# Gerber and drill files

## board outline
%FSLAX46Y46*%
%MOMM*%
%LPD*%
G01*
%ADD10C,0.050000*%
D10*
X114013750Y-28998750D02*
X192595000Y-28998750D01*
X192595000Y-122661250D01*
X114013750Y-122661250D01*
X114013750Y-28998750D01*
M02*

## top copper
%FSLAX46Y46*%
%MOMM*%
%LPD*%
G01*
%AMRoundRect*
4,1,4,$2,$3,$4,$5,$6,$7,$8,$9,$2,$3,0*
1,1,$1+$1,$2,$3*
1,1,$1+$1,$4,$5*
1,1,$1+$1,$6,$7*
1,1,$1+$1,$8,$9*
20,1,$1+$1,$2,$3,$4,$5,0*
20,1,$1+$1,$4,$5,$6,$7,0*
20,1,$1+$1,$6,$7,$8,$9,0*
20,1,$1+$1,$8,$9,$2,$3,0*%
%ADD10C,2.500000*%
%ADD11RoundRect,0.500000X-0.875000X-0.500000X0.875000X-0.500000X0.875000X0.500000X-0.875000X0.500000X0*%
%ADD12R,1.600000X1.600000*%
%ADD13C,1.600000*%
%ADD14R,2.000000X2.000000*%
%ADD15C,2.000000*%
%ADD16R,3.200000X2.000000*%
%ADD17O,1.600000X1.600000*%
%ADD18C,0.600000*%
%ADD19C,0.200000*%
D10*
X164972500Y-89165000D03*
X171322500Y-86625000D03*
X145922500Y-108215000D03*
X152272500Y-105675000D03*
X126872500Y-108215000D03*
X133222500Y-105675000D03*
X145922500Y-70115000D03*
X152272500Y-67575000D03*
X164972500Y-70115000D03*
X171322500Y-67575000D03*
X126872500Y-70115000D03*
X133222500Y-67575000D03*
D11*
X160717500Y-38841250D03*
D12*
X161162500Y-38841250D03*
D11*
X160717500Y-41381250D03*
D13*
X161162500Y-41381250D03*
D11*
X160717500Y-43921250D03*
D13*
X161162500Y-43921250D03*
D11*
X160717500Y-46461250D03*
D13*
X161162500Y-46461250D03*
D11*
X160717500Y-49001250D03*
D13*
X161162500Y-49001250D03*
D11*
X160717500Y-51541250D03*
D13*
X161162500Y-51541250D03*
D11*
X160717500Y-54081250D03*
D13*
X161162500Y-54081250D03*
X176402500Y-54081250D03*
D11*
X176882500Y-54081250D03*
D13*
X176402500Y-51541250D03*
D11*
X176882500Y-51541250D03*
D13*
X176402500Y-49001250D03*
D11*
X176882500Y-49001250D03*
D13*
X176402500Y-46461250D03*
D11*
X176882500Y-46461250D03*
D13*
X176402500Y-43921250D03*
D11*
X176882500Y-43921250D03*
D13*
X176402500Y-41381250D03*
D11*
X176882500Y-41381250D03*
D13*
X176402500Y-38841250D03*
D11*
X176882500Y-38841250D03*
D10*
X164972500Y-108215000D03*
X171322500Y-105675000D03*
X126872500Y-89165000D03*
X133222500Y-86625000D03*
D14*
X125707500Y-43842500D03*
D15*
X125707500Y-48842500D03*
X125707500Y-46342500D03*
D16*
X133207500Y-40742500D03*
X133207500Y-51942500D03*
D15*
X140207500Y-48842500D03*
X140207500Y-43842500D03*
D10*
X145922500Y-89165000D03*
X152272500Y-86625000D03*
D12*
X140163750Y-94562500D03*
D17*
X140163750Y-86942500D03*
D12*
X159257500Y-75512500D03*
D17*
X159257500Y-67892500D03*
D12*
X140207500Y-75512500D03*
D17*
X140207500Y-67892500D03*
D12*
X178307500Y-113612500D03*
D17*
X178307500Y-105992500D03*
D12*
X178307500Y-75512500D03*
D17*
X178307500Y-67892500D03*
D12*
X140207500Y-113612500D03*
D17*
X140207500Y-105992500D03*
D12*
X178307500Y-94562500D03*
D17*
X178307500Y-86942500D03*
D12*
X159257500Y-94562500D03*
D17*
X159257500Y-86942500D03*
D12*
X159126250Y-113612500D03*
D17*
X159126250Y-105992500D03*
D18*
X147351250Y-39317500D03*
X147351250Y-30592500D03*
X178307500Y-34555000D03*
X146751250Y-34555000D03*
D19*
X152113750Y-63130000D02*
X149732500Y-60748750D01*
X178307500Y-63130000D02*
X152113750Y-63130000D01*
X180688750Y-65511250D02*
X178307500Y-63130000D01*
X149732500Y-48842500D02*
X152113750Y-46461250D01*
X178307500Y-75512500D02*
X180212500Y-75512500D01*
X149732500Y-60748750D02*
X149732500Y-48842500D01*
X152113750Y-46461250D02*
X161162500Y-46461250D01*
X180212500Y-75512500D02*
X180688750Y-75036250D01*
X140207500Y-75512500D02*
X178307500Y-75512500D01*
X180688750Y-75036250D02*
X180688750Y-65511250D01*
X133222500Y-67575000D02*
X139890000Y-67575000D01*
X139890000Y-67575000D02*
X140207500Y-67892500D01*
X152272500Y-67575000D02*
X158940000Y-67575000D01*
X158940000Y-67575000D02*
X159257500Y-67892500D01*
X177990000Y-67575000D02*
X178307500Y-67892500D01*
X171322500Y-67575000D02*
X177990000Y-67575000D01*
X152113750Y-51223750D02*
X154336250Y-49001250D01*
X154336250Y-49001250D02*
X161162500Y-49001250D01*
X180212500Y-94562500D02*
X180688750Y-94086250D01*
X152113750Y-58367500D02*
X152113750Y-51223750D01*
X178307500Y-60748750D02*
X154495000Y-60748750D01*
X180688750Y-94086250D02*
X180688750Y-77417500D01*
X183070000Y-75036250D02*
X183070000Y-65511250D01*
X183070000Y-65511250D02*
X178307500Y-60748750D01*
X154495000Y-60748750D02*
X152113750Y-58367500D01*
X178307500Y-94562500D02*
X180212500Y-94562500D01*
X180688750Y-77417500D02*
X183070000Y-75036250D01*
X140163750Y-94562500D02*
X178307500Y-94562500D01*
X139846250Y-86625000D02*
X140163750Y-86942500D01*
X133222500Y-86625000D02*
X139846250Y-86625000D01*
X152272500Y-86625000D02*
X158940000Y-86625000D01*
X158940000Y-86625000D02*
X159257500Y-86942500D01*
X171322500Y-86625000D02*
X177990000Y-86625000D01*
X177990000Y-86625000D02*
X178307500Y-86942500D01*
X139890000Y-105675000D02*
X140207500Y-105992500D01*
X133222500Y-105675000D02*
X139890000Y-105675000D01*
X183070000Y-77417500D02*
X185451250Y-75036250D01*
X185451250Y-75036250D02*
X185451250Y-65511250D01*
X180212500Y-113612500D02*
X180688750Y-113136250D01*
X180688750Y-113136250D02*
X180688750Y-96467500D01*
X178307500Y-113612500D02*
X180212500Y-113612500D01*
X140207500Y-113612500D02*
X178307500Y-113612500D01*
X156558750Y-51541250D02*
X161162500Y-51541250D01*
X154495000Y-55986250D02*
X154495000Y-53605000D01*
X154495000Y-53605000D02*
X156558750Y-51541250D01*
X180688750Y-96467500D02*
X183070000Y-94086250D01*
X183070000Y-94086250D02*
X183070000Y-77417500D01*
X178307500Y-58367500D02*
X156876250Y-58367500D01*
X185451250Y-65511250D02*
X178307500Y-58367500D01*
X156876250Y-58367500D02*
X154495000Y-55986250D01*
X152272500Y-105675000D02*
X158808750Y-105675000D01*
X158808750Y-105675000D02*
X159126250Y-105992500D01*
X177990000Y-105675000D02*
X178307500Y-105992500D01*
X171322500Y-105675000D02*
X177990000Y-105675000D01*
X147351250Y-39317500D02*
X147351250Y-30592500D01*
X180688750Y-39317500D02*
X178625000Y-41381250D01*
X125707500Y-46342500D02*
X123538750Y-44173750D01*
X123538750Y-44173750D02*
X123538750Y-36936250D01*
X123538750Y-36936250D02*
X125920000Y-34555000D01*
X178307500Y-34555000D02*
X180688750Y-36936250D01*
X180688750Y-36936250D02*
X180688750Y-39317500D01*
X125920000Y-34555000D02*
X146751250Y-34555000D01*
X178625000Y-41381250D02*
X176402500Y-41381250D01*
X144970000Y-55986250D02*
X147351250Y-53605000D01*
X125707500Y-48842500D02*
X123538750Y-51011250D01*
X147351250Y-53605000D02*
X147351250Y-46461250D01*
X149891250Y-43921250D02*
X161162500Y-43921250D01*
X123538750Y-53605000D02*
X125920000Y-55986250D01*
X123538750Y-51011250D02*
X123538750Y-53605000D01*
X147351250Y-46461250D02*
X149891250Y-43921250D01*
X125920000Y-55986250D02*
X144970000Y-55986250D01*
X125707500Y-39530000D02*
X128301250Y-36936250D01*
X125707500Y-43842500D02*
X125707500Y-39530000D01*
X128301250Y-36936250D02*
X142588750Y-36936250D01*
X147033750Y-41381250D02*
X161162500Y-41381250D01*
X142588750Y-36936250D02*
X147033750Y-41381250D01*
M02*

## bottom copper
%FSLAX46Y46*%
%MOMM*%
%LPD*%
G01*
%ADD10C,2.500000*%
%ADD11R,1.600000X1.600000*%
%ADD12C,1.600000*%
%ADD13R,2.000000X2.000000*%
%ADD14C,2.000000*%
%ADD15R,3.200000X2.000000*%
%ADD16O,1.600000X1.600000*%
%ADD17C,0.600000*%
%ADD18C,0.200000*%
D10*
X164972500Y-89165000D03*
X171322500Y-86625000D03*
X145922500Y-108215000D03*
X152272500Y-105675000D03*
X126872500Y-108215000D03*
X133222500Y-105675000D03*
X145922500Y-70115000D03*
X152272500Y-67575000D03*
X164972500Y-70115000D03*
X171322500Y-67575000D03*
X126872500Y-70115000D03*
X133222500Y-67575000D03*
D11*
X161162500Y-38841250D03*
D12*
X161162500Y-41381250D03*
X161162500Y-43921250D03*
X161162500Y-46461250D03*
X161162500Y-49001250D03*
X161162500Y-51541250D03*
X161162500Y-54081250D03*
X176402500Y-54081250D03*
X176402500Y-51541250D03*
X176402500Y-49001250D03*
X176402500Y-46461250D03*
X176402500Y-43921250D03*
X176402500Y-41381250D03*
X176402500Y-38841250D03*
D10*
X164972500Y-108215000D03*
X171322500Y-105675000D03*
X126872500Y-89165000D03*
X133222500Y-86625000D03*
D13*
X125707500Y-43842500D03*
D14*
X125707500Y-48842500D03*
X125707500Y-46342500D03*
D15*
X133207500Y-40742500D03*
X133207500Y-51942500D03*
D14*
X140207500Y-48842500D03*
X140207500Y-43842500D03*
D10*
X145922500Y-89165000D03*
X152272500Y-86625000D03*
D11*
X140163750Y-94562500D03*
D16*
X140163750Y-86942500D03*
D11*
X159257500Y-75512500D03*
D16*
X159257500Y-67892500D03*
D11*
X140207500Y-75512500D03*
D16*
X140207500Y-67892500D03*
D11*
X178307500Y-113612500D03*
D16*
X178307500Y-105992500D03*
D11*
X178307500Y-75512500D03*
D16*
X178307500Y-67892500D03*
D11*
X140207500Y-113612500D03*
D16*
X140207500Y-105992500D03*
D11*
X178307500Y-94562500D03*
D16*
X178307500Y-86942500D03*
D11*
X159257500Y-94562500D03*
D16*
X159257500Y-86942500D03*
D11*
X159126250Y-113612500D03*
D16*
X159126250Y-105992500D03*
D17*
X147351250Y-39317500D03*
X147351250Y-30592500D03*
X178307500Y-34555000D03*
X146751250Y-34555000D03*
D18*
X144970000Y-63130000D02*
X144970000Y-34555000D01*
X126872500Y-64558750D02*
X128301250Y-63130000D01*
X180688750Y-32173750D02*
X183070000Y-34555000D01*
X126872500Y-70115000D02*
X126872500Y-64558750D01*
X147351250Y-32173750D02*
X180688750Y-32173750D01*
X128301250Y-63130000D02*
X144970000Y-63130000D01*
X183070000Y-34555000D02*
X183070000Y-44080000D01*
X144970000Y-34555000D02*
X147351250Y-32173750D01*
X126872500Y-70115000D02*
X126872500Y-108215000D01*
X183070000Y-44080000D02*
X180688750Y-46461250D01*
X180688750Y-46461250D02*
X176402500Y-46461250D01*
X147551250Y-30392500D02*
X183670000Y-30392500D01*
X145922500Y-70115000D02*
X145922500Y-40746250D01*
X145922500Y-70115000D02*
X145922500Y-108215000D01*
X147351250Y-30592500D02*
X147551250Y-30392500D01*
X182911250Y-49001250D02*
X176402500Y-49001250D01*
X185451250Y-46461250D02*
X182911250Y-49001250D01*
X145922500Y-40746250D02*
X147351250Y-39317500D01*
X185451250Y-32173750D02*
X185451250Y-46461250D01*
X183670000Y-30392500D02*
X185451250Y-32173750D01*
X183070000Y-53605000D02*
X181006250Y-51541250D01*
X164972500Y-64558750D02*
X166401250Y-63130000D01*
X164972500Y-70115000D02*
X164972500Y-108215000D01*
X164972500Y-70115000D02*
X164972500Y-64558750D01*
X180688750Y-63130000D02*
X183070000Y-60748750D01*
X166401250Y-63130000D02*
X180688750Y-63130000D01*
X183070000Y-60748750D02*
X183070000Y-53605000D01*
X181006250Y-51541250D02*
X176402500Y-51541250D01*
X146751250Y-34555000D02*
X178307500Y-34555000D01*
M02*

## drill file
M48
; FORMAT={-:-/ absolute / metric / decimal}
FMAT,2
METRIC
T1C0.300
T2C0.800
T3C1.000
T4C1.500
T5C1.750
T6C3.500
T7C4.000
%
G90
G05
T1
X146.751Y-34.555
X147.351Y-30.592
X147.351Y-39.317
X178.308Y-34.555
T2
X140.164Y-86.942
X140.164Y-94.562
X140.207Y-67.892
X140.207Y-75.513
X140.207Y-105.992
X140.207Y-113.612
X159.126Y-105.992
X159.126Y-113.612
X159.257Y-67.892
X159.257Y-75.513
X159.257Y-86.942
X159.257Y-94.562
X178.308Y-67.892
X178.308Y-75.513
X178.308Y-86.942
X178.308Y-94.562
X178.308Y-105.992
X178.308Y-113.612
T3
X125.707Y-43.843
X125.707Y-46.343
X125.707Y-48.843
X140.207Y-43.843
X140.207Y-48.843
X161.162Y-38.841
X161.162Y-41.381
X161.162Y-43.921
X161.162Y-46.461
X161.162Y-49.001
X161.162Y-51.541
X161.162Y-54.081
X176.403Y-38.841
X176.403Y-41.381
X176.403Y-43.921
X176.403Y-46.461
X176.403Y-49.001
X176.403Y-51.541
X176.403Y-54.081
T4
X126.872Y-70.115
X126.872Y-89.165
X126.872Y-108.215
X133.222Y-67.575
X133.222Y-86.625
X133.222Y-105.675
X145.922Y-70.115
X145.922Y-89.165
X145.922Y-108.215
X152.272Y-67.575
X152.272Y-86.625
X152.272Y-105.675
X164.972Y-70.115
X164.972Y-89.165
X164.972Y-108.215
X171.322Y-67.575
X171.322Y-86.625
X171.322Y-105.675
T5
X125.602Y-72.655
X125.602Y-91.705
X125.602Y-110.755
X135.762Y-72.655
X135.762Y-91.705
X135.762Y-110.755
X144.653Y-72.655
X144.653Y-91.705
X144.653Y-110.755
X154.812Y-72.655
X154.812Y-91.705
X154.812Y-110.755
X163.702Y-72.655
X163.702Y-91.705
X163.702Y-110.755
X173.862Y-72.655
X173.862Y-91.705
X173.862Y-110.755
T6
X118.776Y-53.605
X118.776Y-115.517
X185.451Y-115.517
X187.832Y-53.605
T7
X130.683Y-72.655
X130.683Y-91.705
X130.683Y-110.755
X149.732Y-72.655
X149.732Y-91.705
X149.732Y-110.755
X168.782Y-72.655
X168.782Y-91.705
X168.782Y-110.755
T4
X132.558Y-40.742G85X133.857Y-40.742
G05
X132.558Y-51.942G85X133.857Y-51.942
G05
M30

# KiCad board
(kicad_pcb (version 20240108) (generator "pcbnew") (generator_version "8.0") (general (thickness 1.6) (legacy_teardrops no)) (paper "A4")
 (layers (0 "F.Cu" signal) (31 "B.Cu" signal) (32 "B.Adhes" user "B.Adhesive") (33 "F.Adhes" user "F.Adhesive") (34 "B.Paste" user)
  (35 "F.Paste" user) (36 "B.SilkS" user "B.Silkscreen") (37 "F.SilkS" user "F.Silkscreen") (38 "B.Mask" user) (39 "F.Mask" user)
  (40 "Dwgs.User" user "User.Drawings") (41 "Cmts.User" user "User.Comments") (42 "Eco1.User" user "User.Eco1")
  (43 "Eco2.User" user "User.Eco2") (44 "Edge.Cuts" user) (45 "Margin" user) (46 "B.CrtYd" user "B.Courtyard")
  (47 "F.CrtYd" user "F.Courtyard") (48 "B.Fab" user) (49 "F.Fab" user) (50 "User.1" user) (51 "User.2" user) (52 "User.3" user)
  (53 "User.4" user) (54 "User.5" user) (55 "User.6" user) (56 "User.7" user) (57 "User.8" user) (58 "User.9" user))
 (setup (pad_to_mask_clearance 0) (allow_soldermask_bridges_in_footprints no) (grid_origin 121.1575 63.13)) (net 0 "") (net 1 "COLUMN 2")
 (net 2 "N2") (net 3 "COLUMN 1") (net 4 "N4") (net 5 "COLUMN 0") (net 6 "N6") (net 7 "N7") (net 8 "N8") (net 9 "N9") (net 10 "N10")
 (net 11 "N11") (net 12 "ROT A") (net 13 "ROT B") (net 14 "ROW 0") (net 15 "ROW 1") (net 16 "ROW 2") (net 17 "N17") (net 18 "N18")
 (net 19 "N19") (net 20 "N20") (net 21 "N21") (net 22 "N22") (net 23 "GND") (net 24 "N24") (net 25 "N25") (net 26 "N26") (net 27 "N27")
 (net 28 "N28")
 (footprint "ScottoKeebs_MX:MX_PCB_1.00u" (layer "F.Cu") (at 168.7825 91.705)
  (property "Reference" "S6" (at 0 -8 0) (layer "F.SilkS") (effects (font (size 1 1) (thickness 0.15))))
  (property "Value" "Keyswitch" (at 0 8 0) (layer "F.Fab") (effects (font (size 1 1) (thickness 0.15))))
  (pad "" np_thru_hole circle (at -5.08 0) (size 1.75 1.75) (drill 1.75) (layers "*.Cu" "*.Mask"))
  (pad "" np_thru_hole circle (at 0 0) (size 4 4) (drill 4) (layers "*.Cu" "*.Mask"))
  (pad "" np_thru_hole circle (at 5.08 0) (size 1.75 1.75) (drill 1.75) (layers "*.Cu" "*.Mask"))
  (pad "1" thru_hole circle (at -3.81 -2.54) (size 2.5 2.5) (drill 1.5) (layers "*.Cu" "*.Mask") (remove_unused_layers no)
   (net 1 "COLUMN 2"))
  (pad "2" thru_hole circle (at 2.54 -5.08) (size 2.5 2.5) (drill 1.5) (layers "*.Cu" "*.Mask") (remove_unused_layers no) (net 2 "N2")))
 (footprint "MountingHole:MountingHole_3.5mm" (layer "F.Cu") (at 118.77625 53.605)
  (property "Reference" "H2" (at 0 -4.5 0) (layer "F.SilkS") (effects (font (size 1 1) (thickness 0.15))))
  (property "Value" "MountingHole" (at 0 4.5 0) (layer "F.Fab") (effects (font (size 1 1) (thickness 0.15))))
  (pad "" np_thru_hole circle (at 0 0) (size 3.5 3.5) (drill 3.5) (layers "*.Cu" "*.Mask")))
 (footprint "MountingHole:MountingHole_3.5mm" (layer "F.Cu") (at 118.77625 115.5175)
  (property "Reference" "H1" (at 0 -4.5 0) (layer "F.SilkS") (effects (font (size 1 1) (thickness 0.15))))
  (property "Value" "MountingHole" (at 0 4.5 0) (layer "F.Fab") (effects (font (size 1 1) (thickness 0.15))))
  (pad "" np_thru_hole circle (at 0 0) (size 3.5 3.5) (drill 3.5) (layers "*.Cu" "*.Mask")))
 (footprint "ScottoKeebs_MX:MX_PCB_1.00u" (layer "F.Cu") (at 149.7325 110.755)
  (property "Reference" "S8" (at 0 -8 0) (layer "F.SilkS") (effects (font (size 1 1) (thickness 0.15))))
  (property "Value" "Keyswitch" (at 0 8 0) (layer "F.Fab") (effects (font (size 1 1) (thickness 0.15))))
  (pad "" np_thru_hole circle (at -5.08 0) (size 1.75 1.75) (drill 1.75) (layers "*.Cu" "*.Mask"))
  (pad "" np_thru_hole circle (at 0 0) (size 4 4) (drill 4) (layers "*.Cu" "*.Mask"))
  (pad "" np_thru_hole circle (at 5.08 0) (size 1.75 1.75) (drill 1.75) (layers "*.Cu" "*.Mask"))
  (pad "1" thru_hole circle (at -3.81 -2.54) (size 2.5 2.5) (drill 1.5) (layers "*.Cu" "*.Mask") (remove_unused_layers no)
   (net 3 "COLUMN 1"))
  (pad "2" thru_hole circle (at 2.54 -5.08) (size 2.5 2.5) (drill 1.5) (layers "*.Cu" "*.Mask") (remove_unused_layers no) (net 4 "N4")))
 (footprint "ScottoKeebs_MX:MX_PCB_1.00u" (layer "F.Cu") (at 130.6825 110.755)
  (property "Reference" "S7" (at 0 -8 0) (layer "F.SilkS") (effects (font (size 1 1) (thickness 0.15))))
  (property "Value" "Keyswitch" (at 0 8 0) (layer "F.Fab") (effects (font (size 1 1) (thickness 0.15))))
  (pad "" np_thru_hole circle (at -5.08 0) (size 1.75 1.75) (drill 1.75) (layers "*.Cu" "*.Mask"))
  (pad "" np_thru_hole circle (at 0 0) (size 4 4) (drill 4) (layers "*.Cu" "*.Mask"))
  (pad "" np_thru_hole circle (at 5.08 0) (size 1.75 1.75) (drill 1.75) (layers "*.Cu" "*.Mask"))
  (pad "1" thru_hole circle (at -3.81 -2.54) (size 2.5 2.5) (drill 1.5) (layers "*.Cu" "*.Mask") (remove_unused_layers no)
   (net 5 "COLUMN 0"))
  (pad "2" thru_hole circle (at 2.54 -5.08) (size 2.5 2.5) (drill 1.5) (layers "*.Cu" "*.Mask") (remove_unused_layers no) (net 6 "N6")))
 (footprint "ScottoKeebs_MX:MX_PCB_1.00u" (layer "F.Cu") (at 149.7325 72.655)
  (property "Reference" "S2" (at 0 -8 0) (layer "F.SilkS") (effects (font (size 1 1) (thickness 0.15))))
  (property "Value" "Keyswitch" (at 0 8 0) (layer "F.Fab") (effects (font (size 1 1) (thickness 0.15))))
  (pad "" np_thru_hole circle (at -5.08 0) (size 1.75 1.75) (drill 1.75) (layers "*.Cu" "*.Mask"))
  (pad "" np_thru_hole circle (at 0 0) (size 4 4) (drill 4) (layers "*.Cu" "*.Mask"))
  (pad "" np_thru_hole circle (at 5.08 0) (size 1.75 1.75) (drill 1.75) (layers "*.Cu" "*.Mask"))
  (pad "1" thru_hole circle (at -3.81 -2.54) (size 2.5 2.5) (drill 1.5) (layers "*.Cu" "*.Mask") (remove_unused_layers no)
   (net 3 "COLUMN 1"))
  (pad "2" thru_hole circle (at 2.54 -5.08) (size 2.5 2.5) (drill 1.5) (layers "*.Cu" "*.Mask") (remove_unused_layers no) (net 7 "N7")))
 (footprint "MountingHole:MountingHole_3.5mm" (layer "F.Cu") (at 187.8325 53.605)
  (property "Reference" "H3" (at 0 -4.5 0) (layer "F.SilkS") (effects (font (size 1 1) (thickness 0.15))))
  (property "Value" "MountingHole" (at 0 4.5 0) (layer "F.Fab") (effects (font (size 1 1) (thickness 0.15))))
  (pad "" np_thru_hole circle (at 0 0) (size 3.5 3.5) (drill 3.5) (layers "*.Cu" "*.Mask")))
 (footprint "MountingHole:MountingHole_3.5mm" (layer "F.Cu") (at 185.45125 115.5175)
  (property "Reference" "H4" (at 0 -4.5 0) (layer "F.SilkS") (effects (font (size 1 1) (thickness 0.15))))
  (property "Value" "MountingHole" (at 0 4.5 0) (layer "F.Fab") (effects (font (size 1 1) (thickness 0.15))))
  (pad "" np_thru_hole circle (at 0 0) (size 3.5 3.5) (drill 3.5) (layers "*.Cu" "*.Mask")))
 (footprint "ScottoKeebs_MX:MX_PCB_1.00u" (layer "F.Cu") (at 168.7825 72.655)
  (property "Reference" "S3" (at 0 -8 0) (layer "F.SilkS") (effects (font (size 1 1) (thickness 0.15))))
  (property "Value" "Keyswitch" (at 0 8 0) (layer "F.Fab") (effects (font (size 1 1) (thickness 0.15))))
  (pad "" np_thru_hole circle (at -5.08 0) (size 1.75 1.75) (drill 1.75) (layers "*.Cu" "*.Mask"))
  (pad "" np_thru_hole circle (at 0 0) (size 4 4) (drill 4) (layers "*.Cu" "*.Mask"))
  (pad "" np_thru_hole circle (at 5.08 0) (size 1.75 1.75) (drill 1.75) (layers "*.Cu" "*.Mask"))
  (pad "1" thru_hole circle (at -3.81 -2.54) (size 2.5 2.5) (drill 1.5) (layers "*.Cu" "*.Mask") (remove_unused_layers no)
   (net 1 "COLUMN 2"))
  (pad "2" thru_hole circle (at 2.54 -5.08) (size 2.5 2.5) (drill 1.5) (layers "*.Cu" "*.Mask") (remove_unused_layers no) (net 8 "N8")))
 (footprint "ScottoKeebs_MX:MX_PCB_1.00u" (layer "F.Cu") (at 130.6825 72.655)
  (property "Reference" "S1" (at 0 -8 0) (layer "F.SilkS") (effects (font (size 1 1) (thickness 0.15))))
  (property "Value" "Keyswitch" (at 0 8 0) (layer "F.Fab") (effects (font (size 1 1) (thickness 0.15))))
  (pad "" np_thru_hole circle (at -5.08 0) (size 1.75 1.75) (drill 1.75) (layers "*.Cu" "*.Mask"))
  (pad "" np_thru_hole circle (at 0 0) (size 4 4) (drill 4) (layers "*.Cu" "*.Mask"))
  (pad "" np_thru_hole circle (at 5.08 0) (size 1.75 1.75) (drill 1.75) (layers "*.Cu" "*.Mask"))
  (pad "1" thru_hole circle (at -3.81 -2.54) (size 2.5 2.5) (drill 1.5) (layers "*.Cu" "*.Mask") (remove_unused_layers no)
   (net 5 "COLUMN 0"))
  (pad "2" thru_hole circle (at 2.54 -5.08) (size 2.5 2.5) (drill 1.5) (layers "*.Cu" "*.Mask") (remove_unused_layers no) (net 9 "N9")))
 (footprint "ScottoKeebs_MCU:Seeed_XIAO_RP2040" (layer "F.Cu") (at 168.7825 46.46125)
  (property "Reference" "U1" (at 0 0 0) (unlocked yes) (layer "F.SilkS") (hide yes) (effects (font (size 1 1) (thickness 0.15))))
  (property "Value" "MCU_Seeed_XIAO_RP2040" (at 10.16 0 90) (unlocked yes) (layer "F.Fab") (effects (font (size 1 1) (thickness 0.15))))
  (pad "1" smd roundrect (at -8.065 -7.62) (size 2.75 2) (layers "F.Cu" "F.Paste" "F.Mask") (roundrect_rratio 0.25) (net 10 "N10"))
  (pad "1" thru_hole rect (at -7.62 -7.62 90) (size 1.6 1.6) (drill 1) (layers "*.Cu" "*.Mask") (remove_unused_layers no) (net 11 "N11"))
  (pad "2" smd roundrect (at -8.065 -5.08) (size 2.75 2) (layers "F.Cu" "F.Paste" "F.Mask") (roundrect_rratio 0.25) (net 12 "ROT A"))
  (pad "2" thru_hole circle (at -7.62 -5.08 90) (size 1.6 1.6) (drill 1) (layers "*.Cu" "*.Mask") (remove_unused_layers no) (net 12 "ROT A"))
  (pad "3" smd roundrect (at -8.065 -2.54) (size 2.75 2) (layers "F.Cu" "F.Paste" "F.Mask") (roundrect_rratio 0.25) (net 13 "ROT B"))
  (pad "3" thru_hole circle (at -7.62 -2.54 90) (size 1.6 1.6) (drill 1) (layers "*.Cu" "*.Mask") (remove_unused_layers no) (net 13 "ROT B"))
  (pad "4" smd roundrect (at -8.065 0) (size 2.75 2) (layers "F.Cu" "F.Paste" "F.Mask") (roundrect_rratio 0.25) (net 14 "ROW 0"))
  (pad "4" thru_hole circle (at -7.62 0 90) (size 1.6 1.6) (drill 1) (layers "*.Cu" "*.Mask") (remove_unused_layers no) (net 14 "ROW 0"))
  (pad "5" smd roundrect (at -8.065 2.54) (size 2.75 2) (layers "F.Cu" "F.Paste" "F.Mask") (roundrect_rratio 0.25) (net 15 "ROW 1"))
  (pad "5" thru_hole circle (at -7.62 2.54 90) (size 1.6 1.6) (drill 1) (layers "*.Cu" "*.Mask") (remove_unused_layers no) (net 15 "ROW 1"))
  (pad "6" smd roundrect (at -8.065 5.08) (size 2.75 2) (layers "F.Cu" "F.Paste" "F.Mask") (roundrect_rratio 0.25) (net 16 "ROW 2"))
  (pad "6" thru_hole circle (at -7.62 5.08 90) (size 1.6 1.6) (drill 1) (layers "*.Cu" "*.Mask") (remove_unused_layers no) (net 16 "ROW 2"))
  (pad "7" smd roundrect (at -8.065 7.62) (size 2.75 2) (layers "F.Cu" "F.Paste" "F.Mask") (roundrect_rratio 0.25) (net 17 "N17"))
  (pad "7" thru_hole circle (at -7.62 7.62 90) (size 1.6 1.6) (drill 1) (layers "*.Cu" "*.Mask") (remove_unused_layers no) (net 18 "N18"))
  (pad "8" thru_hole circle (at 7.62 7.62 90) (size 1.6 1.6) (drill 1) (layers "*.Cu" "*.Mask") (remove_unused_layers no) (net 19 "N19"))
  (pad "8" smd roundrect (at 8.1 7.62) (size 2.75 2) (layers "F.Cu" "F.Paste" "F.Mask") (roundrect_rratio 0.25) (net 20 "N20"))
  (pad "9" thru_hole circle (at 7.62 5.08 90) (size 1.6 1.6) (drill 1) (layers "*.Cu" "*.Mask") (remove_unused_layers no) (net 1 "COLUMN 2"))
  (pad "9" smd roundrect (at 8.1 5.08) (size 2.75 2) (layers "F.Cu" "F.Paste" "F.Mask") (roundrect_rratio 0.25) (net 1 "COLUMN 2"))
  (pad "10" thru_hole circle (at 7.62 2.54 90) (size 1.6 1.6) (drill 1) (layers "*.Cu" "*.Mask") (remove_unused_layers no)
   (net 3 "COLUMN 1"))
  (pad "10" smd roundrect (at 8.1 2.54) (size 2.75 2) (layers "F.Cu" "F.Paste" "F.Mask") (roundrect_rratio 0.25) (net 3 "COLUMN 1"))
  (pad "11" thru_hole circle (at 7.62 0 90) (size 1.6 1.6) (drill 1) (layers "*.Cu" "*.Mask") (remove_unused_layers no) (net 5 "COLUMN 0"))
  (pad "11" smd roundrect (at 8.1 0) (size 2.75 2) (layers "F.Cu" "F.Paste" "F.Mask") (roundrect_rratio 0.25) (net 5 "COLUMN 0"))
  (pad "12" thru_hole circle (at 7.62 -2.54 90) (size 1.6 1.6) (drill 1) (layers "*.Cu" "*.Mask") (remove_unused_layers no) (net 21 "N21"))
  (pad "12" smd roundrect (at 8.1 -2.54) (size 2.75 2) (layers "F.Cu" "F.Paste" "F.Mask") (roundrect_rratio 0.25) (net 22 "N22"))
  (pad "13" thru_hole circle (at 7.62 -5.08 90) (size 1.6 1.6) (drill 1) (layers "*.Cu" "*.Mask") (remove_unused_layers no) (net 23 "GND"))
  (pad "13" smd roundrect (at 8.1 -5.08) (size 2.75 2) (layers "F.Cu" "F.Paste" "F.Mask") (roundrect_rratio 0.25) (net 23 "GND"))
  (pad "14" thru_hole circle (at 7.62 -7.62 90) (size 1.6 1.6) (drill 1) (layers "*.Cu" "*.Mask") (remove_unused_layers no) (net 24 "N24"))
  (pad "14" smd roundrect (at 8.1 -7.62) (size 2.75 2) (layers "F.Cu" "F.Paste" "F.Mask") (roundrect_rratio 0.25) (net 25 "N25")))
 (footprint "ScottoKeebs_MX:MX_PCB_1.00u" (layer "F.Cu") (at 168.7825 110.755)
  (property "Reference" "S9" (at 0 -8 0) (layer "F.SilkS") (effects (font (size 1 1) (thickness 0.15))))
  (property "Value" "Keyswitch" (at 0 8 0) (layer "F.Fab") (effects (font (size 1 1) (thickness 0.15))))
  (pad "" np_thru_hole circle (at -5.08 0) (size 1.75 1.75) (drill 1.75) (layers "*.Cu" "*.Mask"))
  (pad "" np_thru_hole circle (at 0 0) (size 4 4) (drill 4) (layers "*.Cu" "*.Mask"))
  (pad "" np_thru_hole circle (at 5.08 0) (size 1.75 1.75) (drill 1.75) (layers "*.Cu" "*.Mask"))
  (pad "1" thru_hole circle (at -3.81 -2.54) (size 2.5 2.5) (drill 1.5) (layers "*.Cu" "*.Mask") (remove_unused_layers no)
   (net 1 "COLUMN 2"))
  (pad "2" thru_hole circle (at 2.54 -5.08) (size 2.5 2.5) (drill 1.5) (layers "*.Cu" "*.Mask") (remove_unused_layers no) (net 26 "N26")))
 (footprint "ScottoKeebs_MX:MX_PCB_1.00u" (layer "F.Cu") (at 130.6825 91.705)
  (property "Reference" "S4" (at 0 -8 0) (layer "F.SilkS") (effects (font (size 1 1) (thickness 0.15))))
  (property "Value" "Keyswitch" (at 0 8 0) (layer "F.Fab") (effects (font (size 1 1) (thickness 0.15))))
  (pad "" np_thru_hole circle (at -5.08 0) (size 1.75 1.75) (drill 1.75) (layers "*.Cu" "*.Mask"))
  (pad "" np_thru_hole circle (at 0 0) (size 4 4) (drill 4) (layers "*.Cu" "*.Mask"))
  (pad "" np_thru_hole circle (at 5.08 0) (size 1.75 1.75) (drill 1.75) (layers "*.Cu" "*.Mask"))
  (pad "1" thru_hole circle (at -3.81 -2.54) (size 2.5 2.5) (drill 1.5) (layers "*.Cu" "*.Mask") (remove_unused_layers no)
   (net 5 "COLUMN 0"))
  (pad "2" thru_hole circle (at 2.54 -5.08) (size 2.5 2.5) (drill 1.5) (layers "*.Cu" "*.Mask") (remove_unused_layers no) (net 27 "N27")))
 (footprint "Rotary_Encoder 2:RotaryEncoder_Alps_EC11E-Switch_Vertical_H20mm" (layer "F.Cu") (at 125.7075 43.8425)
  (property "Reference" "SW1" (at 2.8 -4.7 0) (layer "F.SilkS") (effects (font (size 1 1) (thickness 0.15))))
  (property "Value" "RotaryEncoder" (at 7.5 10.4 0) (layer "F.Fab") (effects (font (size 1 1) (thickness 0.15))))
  (pad "A" thru_hole rect (at 0 0) (size 2 2) (drill 1) (layers "*.Cu" "*.Mask") (remove_unused_layers no) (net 12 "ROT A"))
  (pad "B" thru_hole circle (at 0 5) (size 2 2) (drill 1) (layers "*.Cu" "*.Mask") (remove_unused_layers no) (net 13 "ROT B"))
  (pad "C" thru_hole circle (at 0 2.5) (size 2 2) (drill 1) (layers "*.Cu" "*.Mask") (remove_unused_layers no) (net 23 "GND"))
  (pad "MP" thru_hole rect (at 7.5 -3.1) (size 3.2 2) (drill oval 2.8 1.5) (layers "*.Cu" "*.Mask") (remove_unused_layers no))
  (pad "MP" thru_hole rect (at 7.5 8.1) (size 3.2 2) (drill oval 2.8 1.5) (layers "*.Cu" "*.Mask") (remove_unused_layers no))
  (pad "S1" thru_hole circle (at 14.5 5) (size 2 2) (drill 1) (layers "*.Cu" "*.Mask") (remove_unused_layers no))
  (pad "S2" thru_hole circle (at 14.5 0) (size 2 2) (drill 1) (layers "*.Cu" "*.Mask") (remove_unused_layers no)))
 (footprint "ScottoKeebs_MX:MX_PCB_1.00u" (layer "F.Cu") (at 149.7325 91.705)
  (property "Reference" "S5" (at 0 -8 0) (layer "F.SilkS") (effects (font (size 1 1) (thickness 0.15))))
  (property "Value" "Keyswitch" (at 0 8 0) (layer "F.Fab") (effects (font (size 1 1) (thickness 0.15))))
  (pad "" np_thru_hole circle (at -5.08 0) (size 1.75 1.75) (drill 1.75) (layers "*.Cu" "*.Mask"))
  (pad "" np_thru_hole circle (at 0 0) (size 4 4) (drill 4) (layers "*.Cu" "*.Mask"))
  (pad "" np_thru_hole circle (at 5.08 0) (size 1.75 1.75) (drill 1.75) (layers "*.Cu" "*.Mask"))
  (pad "1" thru_hole circle (at -3.81 -2.54) (size 2.5 2.5) (drill 1.5) (layers "*.Cu" "*.Mask") (remove_unused_layers no)
   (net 3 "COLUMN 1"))
  (pad "2" thru_hole circle (at 2.54 -5.08) (size 2.5 2.5) (drill 1.5) (layers "*.Cu" "*.Mask") (remove_unused_layers no) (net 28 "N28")))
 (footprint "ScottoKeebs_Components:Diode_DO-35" (layer "B.Cu") (at 140.16375 94.5625 90)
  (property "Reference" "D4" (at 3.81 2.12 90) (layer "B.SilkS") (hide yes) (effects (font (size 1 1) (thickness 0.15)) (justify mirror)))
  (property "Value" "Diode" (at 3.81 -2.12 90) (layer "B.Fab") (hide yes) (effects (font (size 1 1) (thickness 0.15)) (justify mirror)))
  (pad "1" thru_hole rect (at 0 0 90) (size 1.6 1.6) (drill 0.8) (layers "*.Cu" "*.Mask") (remove_unused_layers no) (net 15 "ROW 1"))
  (pad "2" thru_hole oval (at 7.62 0 90) (size 1.6 1.6) (drill 0.8) (layers "*.Cu" "*.Mask") (remove_unused_layers no) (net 27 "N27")))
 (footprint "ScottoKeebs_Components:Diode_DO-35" (layer "B.Cu") (at 159.2575 75.5125 90)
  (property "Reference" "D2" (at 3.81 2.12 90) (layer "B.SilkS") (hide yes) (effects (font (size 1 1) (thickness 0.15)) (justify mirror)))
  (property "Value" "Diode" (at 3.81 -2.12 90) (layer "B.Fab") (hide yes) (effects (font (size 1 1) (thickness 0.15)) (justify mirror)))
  (pad "1" thru_hole rect (at 0 0 90) (size 1.6 1.6) (drill 0.8) (layers "*.Cu" "*.Mask") (remove_unused_layers no) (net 14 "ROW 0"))
  (pad "2" thru_hole oval (at 7.62 0 90) (size 1.6 1.6) (drill 0.8) (layers "*.Cu" "*.Mask") (remove_unused_layers no) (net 7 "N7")))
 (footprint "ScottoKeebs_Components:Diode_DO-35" (layer "B.Cu") (at 140.2075 75.5125 90)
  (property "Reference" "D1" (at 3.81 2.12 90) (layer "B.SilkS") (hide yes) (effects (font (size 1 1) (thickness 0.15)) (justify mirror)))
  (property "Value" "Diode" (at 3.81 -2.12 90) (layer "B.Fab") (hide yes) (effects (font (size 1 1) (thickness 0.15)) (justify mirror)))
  (pad "1" thru_hole rect (at 0 0 90) (size 1.6 1.6) (drill 0.8) (layers "*.Cu" "*.Mask") (remove_unused_layers no) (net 14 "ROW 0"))
  (pad "2" thru_hole oval (at 7.62 0 90) (size 1.6 1.6) (drill 0.8) (layers "*.Cu" "*.Mask") (remove_unused_layers no) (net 9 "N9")))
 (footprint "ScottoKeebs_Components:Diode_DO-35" (layer "B.Cu") (at 178.3075 113.6125 90)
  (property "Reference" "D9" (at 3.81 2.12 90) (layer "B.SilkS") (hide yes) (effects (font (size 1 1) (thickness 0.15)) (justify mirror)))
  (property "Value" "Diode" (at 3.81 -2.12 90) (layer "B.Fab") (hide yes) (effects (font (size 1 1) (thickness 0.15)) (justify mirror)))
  (pad "1" thru_hole rect (at 0 0 90) (size 1.6 1.6) (drill 0.8) (layers "*.Cu" "*.Mask") (remove_unused_layers no) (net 16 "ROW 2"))
  (pad "2" thru_hole oval (at 7.62 0 90) (size 1.6 1.6) (drill 0.8) (layers "*.Cu" "*.Mask") (remove_unused_layers no) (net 26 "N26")))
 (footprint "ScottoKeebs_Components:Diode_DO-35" (layer "B.Cu") (at 178.3075 75.5125 90)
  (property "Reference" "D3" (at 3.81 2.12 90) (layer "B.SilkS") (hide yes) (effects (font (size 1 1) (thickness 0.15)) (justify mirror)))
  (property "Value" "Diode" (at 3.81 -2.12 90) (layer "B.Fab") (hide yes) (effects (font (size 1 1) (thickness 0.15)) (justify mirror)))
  (pad "1" thru_hole rect (at 0 0 90) (size 1.6 1.6) (drill 0.8) (layers "*.Cu" "*.Mask") (remove_unused_layers no) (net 14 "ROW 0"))
  (pad "2" thru_hole oval (at 7.62 0 90) (size 1.6 1.6) (drill 0.8) (layers "*.Cu" "*.Mask") (remove_unused_layers no) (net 8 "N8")))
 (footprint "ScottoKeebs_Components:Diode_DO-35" (layer "B.Cu") (at 140.2075 113.6125 90)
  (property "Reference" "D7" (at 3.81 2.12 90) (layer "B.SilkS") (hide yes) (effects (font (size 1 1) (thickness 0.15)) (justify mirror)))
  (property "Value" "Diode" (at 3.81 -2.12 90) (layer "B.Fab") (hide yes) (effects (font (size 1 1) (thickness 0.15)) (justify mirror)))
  (pad "1" thru_hole rect (at 0 0 90) (size 1.6 1.6) (drill 0.8) (layers "*.Cu" "*.Mask") (remove_unused_layers no) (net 16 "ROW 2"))
  (pad "2" thru_hole oval (at 7.62 0 90) (size 1.6 1.6) (drill 0.8) (layers "*.Cu" "*.Mask") (remove_unused_layers no) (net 6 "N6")))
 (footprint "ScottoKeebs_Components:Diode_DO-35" (layer "B.Cu") (at 178.3075 94.5625 90)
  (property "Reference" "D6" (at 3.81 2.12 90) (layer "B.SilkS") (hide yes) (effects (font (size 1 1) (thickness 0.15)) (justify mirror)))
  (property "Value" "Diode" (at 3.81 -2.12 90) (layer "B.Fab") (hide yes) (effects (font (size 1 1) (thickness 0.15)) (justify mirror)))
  (pad "1" thru_hole rect (at 0 0 90) (size 1.6 1.6) (drill 0.8) (layers "*.Cu" "*.Mask") (remove_unused_layers no) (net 15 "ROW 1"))
  (pad "2" thru_hole oval (at 7.62 0 90) (size 1.6 1.6) (drill 0.8) (layers "*.Cu" "*.Mask") (remove_unused_layers no) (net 2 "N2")))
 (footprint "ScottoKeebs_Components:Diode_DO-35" (layer "B.Cu") (at 159.2575 94.5625 90)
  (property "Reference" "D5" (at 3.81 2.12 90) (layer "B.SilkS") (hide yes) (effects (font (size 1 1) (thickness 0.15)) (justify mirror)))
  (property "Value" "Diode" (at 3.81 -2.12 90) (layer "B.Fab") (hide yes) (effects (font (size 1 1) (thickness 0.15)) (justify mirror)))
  (pad "1" thru_hole rect (at 0 0 90) (size 1.6 1.6) (drill 0.8) (layers "*.Cu" "*.Mask") (remove_unused_layers no) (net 15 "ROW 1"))
  (pad "2" thru_hole oval (at 7.62 0 90) (size 1.6 1.6) (drill 0.8) (layers "*.Cu" "*.Mask") (remove_unused_layers no) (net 28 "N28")))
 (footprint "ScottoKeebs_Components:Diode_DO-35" (layer "B.Cu") (at 159.12625 113.6125 90)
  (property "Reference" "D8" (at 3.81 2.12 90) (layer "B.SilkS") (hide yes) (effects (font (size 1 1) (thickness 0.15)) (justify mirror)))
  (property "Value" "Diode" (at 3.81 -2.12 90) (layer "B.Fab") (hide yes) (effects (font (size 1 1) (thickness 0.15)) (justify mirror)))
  (pad "1" thru_hole rect (at 0 0 90) (size 1.6 1.6) (drill 0.8) (layers "*.Cu" "*.Mask") (remove_unused_layers no) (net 16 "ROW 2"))
  (pad "2" thru_hole oval (at 7.62 0 90) (size 1.6 1.6) (drill 0.8) (layers "*.Cu" "*.Mask") (remove_unused_layers no) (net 4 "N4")))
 (gr_rect (start 114.01375 28.99875) (end 192.595 122.66125) (stroke (width 0.05) (type default)) (fill none) (layer "Edge.Cuts"))
 (segment (start 152.11375 63.13) (end 149.7325 60.74875) (width 0.2) (layer "F.Cu") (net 14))
 (segment (start 178.3075 63.13) (end 152.11375 63.13) (width 0.2) (layer "F.Cu") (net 14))
 (segment (start 180.68875 65.51125) (end 178.3075 63.13) (width 0.2) (layer "F.Cu") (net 14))
 (segment (start 149.7325 48.8425) (end 152.11375 46.46125) (width 0.2) (layer "F.Cu") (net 14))
 (segment (start 178.3075 75.5125) (end 180.2125 75.5125) (width 0.2) (layer "F.Cu") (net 14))
 (segment (start 149.7325 60.74875) (end 149.7325 48.8425) (width 0.2) (layer "F.Cu") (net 14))
 (segment (start 152.11375 46.46125) (end 161.1625 46.46125) (width 0.2) (layer "F.Cu") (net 14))
 (segment (start 180.2125 75.5125) (end 180.68875 75.03625) (width 0.2) (layer "F.Cu") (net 14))
 (segment (start 140.2075 75.5125) (end 178.3075 75.5125) (width 0.2) (layer "F.Cu") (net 14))
 (segment (start 180.68875 75.03625) (end 180.68875 65.51125) (width 0.2) (layer "F.Cu") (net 14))
 (segment (start 133.2225 67.575) (end 139.89 67.575) (width 0.2) (layer "F.Cu") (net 9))
 (segment (start 139.89 67.575) (end 140.2075 67.8925) (width 0.2) (layer "F.Cu") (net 9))
 (segment (start 152.2725 67.575) (end 158.94 67.575) (width 0.2) (layer "F.Cu") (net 7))
 (segment (start 158.94 67.575) (end 159.2575 67.8925) (width 0.2) (layer "F.Cu") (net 7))
 (segment (start 177.99 67.575) (end 178.3075 67.8925) (width 0.2) (layer "F.Cu") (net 8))
 (segment (start 171.3225 67.575) (end 177.99 67.575) (width 0.2) (layer "F.Cu") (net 8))
 (segment (start 152.11375 51.22375) (end 154.33625 49.00125) (width 0.2) (layer "F.Cu") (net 15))
 (segment (start 154.33625 49.00125) (end 161.1625 49.00125) (width 0.2) (layer "F.Cu") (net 15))
 (segment (start 180.2125 94.5625) (end 180.68875 94.08625) (width 0.2) (layer "F.Cu") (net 15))
 (segment (start 152.11375 58.3675) (end 152.11375 51.22375) (width 0.2) (layer "F.Cu") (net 15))
 (segment (start 178.3075 60.74875) (end 154.495 60.74875) (width 0.2) (layer "F.Cu") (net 15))
 (segment (start 180.68875 94.08625) (end 180.68875 77.4175) (width 0.2) (layer "F.Cu") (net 15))
 (segment (start 183.07 75.03625) (end 183.07 65.51125) (width 0.2) (layer "F.Cu") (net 15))
 (segment (start 183.07 65.51125) (end 178.3075 60.74875) (width 0.2) (layer "F.Cu") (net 15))
 (segment (start 154.495 60.74875) (end 152.11375 58.3675) (width 0.2) (layer "F.Cu") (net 15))
 (segment (start 178.3075 94.5625) (end 180.2125 94.5625) (width 0.2) (layer "F.Cu") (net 15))
 (segment (start 180.68875 77.4175) (end 183.07 75.03625) (width 0.2) (layer "F.Cu") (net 15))
 (segment (start 140.16375 94.5625) (end 178.3075 94.5625) (width 0.2) (layer "F.Cu") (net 15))
 (segment (start 139.84625 86.625) (end 140.16375 86.9425) (width 0.2) (layer "F.Cu") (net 27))
 (segment (start 133.2225 86.625) (end 139.84625 86.625) (width 0.2) (layer "F.Cu") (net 27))
 (segment (start 152.2725 86.625) (end 158.94 86.625) (width 0.2) (layer "F.Cu") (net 28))
 (segment (start 158.94 86.625) (end 159.2575 86.9425) (width 0.2) (layer "F.Cu") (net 28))
 (segment (start 171.3225 86.625) (end 177.99 86.625) (width 0.2) (layer "F.Cu") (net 2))
 (segment (start 177.99 86.625) (end 178.3075 86.9425) (width 0.2) (layer "F.Cu") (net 2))
 (segment (start 139.89 105.675) (end 140.2075 105.9925) (width 0.2) (layer "F.Cu") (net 6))
 (segment (start 133.2225 105.675) (end 139.89 105.675) (width 0.2) (layer "F.Cu") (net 6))
 (segment (start 183.07 77.4175) (end 185.45125 75.03625) (width 0.2) (layer "F.Cu") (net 16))
 (segment (start 185.45125 75.03625) (end 185.45125 65.51125) (width 0.2) (layer "F.Cu") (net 16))
 (segment (start 180.2125 113.6125) (end 180.68875 113.13625) (width 0.2) (layer "F.Cu") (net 16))
 (segment (start 180.68875 113.13625) (end 180.68875 96.4675) (width 0.2) (layer "F.Cu") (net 16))
 (segment (start 178.3075 113.6125) (end 180.2125 113.6125) (width 0.2) (layer "F.Cu") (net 16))
 (segment (start 140.2075 113.6125) (end 178.3075 113.6125) (width 0.2) (layer "F.Cu") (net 16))
 (segment (start 156.55875 51.54125) (end 161.1625 51.54125) (width 0.2) (layer "F.Cu") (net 16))
 (segment (start 154.495 55.98625) (end 154.495 53.605) (width 0.2) (layer "F.Cu") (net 16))
 (segment (start 154.495 53.605) (end 156.55875 51.54125) (width 0.2) (layer "F.Cu") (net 16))
 (segment (start 180.68875 96.4675) (end 183.07 94.08625) (width 0.2) (layer "F.Cu") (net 16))
 (segment (start 183.07 94.08625) (end 183.07 77.4175) (width 0.2) (layer "F.Cu") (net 16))
 (segment (start 178.3075 58.3675) (end 156.87625 58.3675) (width 0.2) (layer "F.Cu") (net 16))
 (segment (start 185.45125 65.51125) (end 178.3075 58.3675) (width 0.2) (layer "F.Cu") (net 16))
 (segment (start 156.87625 58.3675) (end 154.495 55.98625) (width 0.2) (layer "F.Cu") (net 16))
 (segment (start 152.2725 105.675) (end 158.80875 105.675) (width 0.2) (layer "F.Cu") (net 4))
 (segment (start 158.80875 105.675) (end 159.12625 105.9925) (width 0.2) (layer "F.Cu") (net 4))
 (segment (start 177.99 105.675) (end 178.3075 105.9925) (width 0.2) (layer "F.Cu") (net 26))
 (segment (start 171.3225 105.675) (end 177.99 105.675) (width 0.2) (layer "F.Cu") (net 26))
 (segment (start 144.97 63.13) (end 144.97 34.555) (width 0.2) (layer "B.Cu") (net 5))
 (segment (start 126.8725 64.55875) (end 128.30125 63.13) (width 0.2) (layer "B.Cu") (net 5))
 (segment (start 180.68875 32.17375) (end 183.07 34.555) (width 0.2) (layer "B.Cu") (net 5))
 (segment (start 126.8725 70.115) (end 126.8725 64.55875) (width 0.2) (layer "B.Cu") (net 5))
 (segment (start 147.35125 32.17375) (end 180.68875 32.17375) (width 0.2) (layer "B.Cu") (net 5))
 (segment (start 128.30125 63.13) (end 144.97 63.13) (width 0.2) (layer "B.Cu") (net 5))
 (segment (start 183.07 34.555) (end 183.07 44.08) (width 0.2) (layer "B.Cu") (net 5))
 (segment (start 144.97 34.555) (end 147.35125 32.17375) (width 0.2) (layer "B.Cu") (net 5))
 (segment (start 126.8725 70.115) (end 126.8725 108.215) (width 0.2) (layer "B.Cu") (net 5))
 (segment (start 183.07 44.08) (end 180.68875 46.46125) (width 0.2) (layer "B.Cu") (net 5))
 (segment (start 180.68875 46.46125) (end 176.4025 46.46125) (width 0.2) (layer "B.Cu") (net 5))
 (segment (start 147.35125 39.3175) (end 147.35125 30.5925) (width 0.2) (layer "F.Cu") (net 3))
 (via (at 147.35125 39.3175) (size 0.6) (drill 0.3) (layers "F.Cu" "B.Cu") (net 3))
 (via (at 147.35125 30.5925) (size 0.6) (drill 0.3) (layers "F.Cu" "B.Cu") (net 3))
 (segment (start 147.55125 30.3925) (end 183.67 30.3925) (width 0.2) (layer "B.Cu") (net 3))
 (segment (start 145.9225 70.115) (end 145.9225 40.74625) (width 0.2) (layer "B.Cu") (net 3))
 (segment (start 145.9225 70.115) (end 145.9225 108.215) (width 0.2) (layer "B.Cu") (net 3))
 (segment (start 147.35125 30.5925) (end 147.55125 30.3925) (width 0.2) (layer "B.Cu") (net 3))
 (segment (start 182.91125 49.00125) (end 176.4025 49.00125) (width 0.2) (layer "B.Cu") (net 3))
 (segment (start 185.45125 46.46125) (end 182.91125 49.00125) (width 0.2) (layer "B.Cu") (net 3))
 (segment (start 145.9225 40.74625) (end 147.35125 39.3175) (width 0.2) (layer "B.Cu") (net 3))
 (segment (start 185.45125 32.17375) (end 185.45125 46.46125) (width 0.2) (layer "B.Cu") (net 3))
 (segment (start 183.67 30.3925) (end 185.45125 32.17375) (width 0.2) (layer "B.Cu") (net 3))
 (segment (start 183.07 53.605) (end 181.00625 51.54125) (width 0.2) (layer "B.Cu") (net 1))
 (segment (start 164.9725 64.55875) (end 166.40125 63.13) (width 0.2) (layer "B.Cu") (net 1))
 (segment (start 164.9725 70.115) (end 164.9725 108.215) (width 0.2) (layer "B.Cu") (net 1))
 (segment (start 164.9725 70.115) (end 164.9725 64.55875) (width 0.2) (layer "B.Cu") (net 1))
 (segment (start 180.68875 63.13) (end 183.07 60.74875) (width 0.2) (layer "B.Cu") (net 1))
 (segment (start 166.40125 63.13) (end 180.68875 63.13) (width 0.2) (layer "B.Cu") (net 1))
 (segment (start 183.07 60.74875) (end 183.07 53.605) (width 0.2) (layer "B.Cu") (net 1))
 (segment (start 181.00625 51.54125) (end 176.4025 51.54125) (width 0.2) (layer "B.Cu") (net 1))
 (segment (start 180.68875 39.3175) (end 178.625 41.38125) (width 0.2) (layer "F.Cu") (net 23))
 (segment (start 125.7075 46.3425) (end 123.53875 44.17375) (width 0.2) (layer "F.Cu") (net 23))
 (segment (start 123.53875 44.17375) (end 123.53875 36.93625) (width 0.2) (layer "F.Cu") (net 23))
 (segment (start 123.53875 36.93625) (end 125.92 34.555) (width 0.2) (layer "F.Cu") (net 23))
 (segment (start 178.3075 34.555) (end 180.68875 36.93625) (width 0.2) (layer "F.Cu") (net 23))
 (segment (start 180.68875 36.93625) (end 180.68875 39.3175) (width 0.2) (layer "F.Cu") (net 23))
 (segment (start 125.92 34.555) (end 146.75125 34.555) (width 0.2) (layer "F.Cu") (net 23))
 (segment (start 178.625 41.38125) (end 176.4025 41.38125) (width 0.2) (layer "F.Cu") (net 23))
 (via (at 178.3075 34.555) (size 0.6) (drill 0.3) (layers "F.Cu" "B.Cu") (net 23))
 (via (at 146.75125 34.555) (size 0.6) (drill 0.3) (layers "F.Cu" "B.Cu") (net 23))
 (segment (start 146.75125 34.555) (end 178.3075 34.555) (width 0.2) (layer "B.Cu") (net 23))
 (segment (start 144.97 55.98625) (end 147.35125 53.605) (width 0.2) (layer "F.Cu") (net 13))
 (segment (start 125.7075 48.8425) (end 123.53875 51.01125) (width 0.2) (layer "F.Cu") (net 13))
 (segment (start 147.35125 53.605) (end 147.35125 46.46125) (width 0.2) (layer "F.Cu") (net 13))
 (segment (start 149.89125 43.92125) (end 161.1625 43.92125) (width 0.2) (layer "F.Cu") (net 13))
 (segment (start 123.53875 53.605) (end 125.92 55.98625) (width 0.2) (layer "F.Cu") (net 13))
 (segment (start 123.53875 51.01125) (end 123.53875 53.605) (width 0.2) (layer "F.Cu") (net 13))
 (segment (start 147.35125 46.46125) (end 149.89125 43.92125) (width 0.2) (layer "F.Cu") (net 13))
 (segment (start 125.92 55.98625) (end 144.97 55.98625) (width 0.2) (layer "F.Cu") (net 13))
 (segment (start 125.7075 39.53) (end 128.30125 36.93625) (width 0.2) (layer "F.Cu") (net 12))
 (segment (start 125.7075 43.8425) (end 125.7075 39.53) (width 0.2) (layer "F.Cu") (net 12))
 (segment (start 128.30125 36.93625) (end 142.58875 36.93625) (width 0.2) (layer "F.Cu") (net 12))
 (segment (start 147.03375 41.38125) (end 161.1625 41.38125) (width 0.2) (layer "F.Cu") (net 12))
 (segment (start 142.58875 36.93625) (end 147.03375 41.38125) (width 0.2) (layer "F.Cu") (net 12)))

